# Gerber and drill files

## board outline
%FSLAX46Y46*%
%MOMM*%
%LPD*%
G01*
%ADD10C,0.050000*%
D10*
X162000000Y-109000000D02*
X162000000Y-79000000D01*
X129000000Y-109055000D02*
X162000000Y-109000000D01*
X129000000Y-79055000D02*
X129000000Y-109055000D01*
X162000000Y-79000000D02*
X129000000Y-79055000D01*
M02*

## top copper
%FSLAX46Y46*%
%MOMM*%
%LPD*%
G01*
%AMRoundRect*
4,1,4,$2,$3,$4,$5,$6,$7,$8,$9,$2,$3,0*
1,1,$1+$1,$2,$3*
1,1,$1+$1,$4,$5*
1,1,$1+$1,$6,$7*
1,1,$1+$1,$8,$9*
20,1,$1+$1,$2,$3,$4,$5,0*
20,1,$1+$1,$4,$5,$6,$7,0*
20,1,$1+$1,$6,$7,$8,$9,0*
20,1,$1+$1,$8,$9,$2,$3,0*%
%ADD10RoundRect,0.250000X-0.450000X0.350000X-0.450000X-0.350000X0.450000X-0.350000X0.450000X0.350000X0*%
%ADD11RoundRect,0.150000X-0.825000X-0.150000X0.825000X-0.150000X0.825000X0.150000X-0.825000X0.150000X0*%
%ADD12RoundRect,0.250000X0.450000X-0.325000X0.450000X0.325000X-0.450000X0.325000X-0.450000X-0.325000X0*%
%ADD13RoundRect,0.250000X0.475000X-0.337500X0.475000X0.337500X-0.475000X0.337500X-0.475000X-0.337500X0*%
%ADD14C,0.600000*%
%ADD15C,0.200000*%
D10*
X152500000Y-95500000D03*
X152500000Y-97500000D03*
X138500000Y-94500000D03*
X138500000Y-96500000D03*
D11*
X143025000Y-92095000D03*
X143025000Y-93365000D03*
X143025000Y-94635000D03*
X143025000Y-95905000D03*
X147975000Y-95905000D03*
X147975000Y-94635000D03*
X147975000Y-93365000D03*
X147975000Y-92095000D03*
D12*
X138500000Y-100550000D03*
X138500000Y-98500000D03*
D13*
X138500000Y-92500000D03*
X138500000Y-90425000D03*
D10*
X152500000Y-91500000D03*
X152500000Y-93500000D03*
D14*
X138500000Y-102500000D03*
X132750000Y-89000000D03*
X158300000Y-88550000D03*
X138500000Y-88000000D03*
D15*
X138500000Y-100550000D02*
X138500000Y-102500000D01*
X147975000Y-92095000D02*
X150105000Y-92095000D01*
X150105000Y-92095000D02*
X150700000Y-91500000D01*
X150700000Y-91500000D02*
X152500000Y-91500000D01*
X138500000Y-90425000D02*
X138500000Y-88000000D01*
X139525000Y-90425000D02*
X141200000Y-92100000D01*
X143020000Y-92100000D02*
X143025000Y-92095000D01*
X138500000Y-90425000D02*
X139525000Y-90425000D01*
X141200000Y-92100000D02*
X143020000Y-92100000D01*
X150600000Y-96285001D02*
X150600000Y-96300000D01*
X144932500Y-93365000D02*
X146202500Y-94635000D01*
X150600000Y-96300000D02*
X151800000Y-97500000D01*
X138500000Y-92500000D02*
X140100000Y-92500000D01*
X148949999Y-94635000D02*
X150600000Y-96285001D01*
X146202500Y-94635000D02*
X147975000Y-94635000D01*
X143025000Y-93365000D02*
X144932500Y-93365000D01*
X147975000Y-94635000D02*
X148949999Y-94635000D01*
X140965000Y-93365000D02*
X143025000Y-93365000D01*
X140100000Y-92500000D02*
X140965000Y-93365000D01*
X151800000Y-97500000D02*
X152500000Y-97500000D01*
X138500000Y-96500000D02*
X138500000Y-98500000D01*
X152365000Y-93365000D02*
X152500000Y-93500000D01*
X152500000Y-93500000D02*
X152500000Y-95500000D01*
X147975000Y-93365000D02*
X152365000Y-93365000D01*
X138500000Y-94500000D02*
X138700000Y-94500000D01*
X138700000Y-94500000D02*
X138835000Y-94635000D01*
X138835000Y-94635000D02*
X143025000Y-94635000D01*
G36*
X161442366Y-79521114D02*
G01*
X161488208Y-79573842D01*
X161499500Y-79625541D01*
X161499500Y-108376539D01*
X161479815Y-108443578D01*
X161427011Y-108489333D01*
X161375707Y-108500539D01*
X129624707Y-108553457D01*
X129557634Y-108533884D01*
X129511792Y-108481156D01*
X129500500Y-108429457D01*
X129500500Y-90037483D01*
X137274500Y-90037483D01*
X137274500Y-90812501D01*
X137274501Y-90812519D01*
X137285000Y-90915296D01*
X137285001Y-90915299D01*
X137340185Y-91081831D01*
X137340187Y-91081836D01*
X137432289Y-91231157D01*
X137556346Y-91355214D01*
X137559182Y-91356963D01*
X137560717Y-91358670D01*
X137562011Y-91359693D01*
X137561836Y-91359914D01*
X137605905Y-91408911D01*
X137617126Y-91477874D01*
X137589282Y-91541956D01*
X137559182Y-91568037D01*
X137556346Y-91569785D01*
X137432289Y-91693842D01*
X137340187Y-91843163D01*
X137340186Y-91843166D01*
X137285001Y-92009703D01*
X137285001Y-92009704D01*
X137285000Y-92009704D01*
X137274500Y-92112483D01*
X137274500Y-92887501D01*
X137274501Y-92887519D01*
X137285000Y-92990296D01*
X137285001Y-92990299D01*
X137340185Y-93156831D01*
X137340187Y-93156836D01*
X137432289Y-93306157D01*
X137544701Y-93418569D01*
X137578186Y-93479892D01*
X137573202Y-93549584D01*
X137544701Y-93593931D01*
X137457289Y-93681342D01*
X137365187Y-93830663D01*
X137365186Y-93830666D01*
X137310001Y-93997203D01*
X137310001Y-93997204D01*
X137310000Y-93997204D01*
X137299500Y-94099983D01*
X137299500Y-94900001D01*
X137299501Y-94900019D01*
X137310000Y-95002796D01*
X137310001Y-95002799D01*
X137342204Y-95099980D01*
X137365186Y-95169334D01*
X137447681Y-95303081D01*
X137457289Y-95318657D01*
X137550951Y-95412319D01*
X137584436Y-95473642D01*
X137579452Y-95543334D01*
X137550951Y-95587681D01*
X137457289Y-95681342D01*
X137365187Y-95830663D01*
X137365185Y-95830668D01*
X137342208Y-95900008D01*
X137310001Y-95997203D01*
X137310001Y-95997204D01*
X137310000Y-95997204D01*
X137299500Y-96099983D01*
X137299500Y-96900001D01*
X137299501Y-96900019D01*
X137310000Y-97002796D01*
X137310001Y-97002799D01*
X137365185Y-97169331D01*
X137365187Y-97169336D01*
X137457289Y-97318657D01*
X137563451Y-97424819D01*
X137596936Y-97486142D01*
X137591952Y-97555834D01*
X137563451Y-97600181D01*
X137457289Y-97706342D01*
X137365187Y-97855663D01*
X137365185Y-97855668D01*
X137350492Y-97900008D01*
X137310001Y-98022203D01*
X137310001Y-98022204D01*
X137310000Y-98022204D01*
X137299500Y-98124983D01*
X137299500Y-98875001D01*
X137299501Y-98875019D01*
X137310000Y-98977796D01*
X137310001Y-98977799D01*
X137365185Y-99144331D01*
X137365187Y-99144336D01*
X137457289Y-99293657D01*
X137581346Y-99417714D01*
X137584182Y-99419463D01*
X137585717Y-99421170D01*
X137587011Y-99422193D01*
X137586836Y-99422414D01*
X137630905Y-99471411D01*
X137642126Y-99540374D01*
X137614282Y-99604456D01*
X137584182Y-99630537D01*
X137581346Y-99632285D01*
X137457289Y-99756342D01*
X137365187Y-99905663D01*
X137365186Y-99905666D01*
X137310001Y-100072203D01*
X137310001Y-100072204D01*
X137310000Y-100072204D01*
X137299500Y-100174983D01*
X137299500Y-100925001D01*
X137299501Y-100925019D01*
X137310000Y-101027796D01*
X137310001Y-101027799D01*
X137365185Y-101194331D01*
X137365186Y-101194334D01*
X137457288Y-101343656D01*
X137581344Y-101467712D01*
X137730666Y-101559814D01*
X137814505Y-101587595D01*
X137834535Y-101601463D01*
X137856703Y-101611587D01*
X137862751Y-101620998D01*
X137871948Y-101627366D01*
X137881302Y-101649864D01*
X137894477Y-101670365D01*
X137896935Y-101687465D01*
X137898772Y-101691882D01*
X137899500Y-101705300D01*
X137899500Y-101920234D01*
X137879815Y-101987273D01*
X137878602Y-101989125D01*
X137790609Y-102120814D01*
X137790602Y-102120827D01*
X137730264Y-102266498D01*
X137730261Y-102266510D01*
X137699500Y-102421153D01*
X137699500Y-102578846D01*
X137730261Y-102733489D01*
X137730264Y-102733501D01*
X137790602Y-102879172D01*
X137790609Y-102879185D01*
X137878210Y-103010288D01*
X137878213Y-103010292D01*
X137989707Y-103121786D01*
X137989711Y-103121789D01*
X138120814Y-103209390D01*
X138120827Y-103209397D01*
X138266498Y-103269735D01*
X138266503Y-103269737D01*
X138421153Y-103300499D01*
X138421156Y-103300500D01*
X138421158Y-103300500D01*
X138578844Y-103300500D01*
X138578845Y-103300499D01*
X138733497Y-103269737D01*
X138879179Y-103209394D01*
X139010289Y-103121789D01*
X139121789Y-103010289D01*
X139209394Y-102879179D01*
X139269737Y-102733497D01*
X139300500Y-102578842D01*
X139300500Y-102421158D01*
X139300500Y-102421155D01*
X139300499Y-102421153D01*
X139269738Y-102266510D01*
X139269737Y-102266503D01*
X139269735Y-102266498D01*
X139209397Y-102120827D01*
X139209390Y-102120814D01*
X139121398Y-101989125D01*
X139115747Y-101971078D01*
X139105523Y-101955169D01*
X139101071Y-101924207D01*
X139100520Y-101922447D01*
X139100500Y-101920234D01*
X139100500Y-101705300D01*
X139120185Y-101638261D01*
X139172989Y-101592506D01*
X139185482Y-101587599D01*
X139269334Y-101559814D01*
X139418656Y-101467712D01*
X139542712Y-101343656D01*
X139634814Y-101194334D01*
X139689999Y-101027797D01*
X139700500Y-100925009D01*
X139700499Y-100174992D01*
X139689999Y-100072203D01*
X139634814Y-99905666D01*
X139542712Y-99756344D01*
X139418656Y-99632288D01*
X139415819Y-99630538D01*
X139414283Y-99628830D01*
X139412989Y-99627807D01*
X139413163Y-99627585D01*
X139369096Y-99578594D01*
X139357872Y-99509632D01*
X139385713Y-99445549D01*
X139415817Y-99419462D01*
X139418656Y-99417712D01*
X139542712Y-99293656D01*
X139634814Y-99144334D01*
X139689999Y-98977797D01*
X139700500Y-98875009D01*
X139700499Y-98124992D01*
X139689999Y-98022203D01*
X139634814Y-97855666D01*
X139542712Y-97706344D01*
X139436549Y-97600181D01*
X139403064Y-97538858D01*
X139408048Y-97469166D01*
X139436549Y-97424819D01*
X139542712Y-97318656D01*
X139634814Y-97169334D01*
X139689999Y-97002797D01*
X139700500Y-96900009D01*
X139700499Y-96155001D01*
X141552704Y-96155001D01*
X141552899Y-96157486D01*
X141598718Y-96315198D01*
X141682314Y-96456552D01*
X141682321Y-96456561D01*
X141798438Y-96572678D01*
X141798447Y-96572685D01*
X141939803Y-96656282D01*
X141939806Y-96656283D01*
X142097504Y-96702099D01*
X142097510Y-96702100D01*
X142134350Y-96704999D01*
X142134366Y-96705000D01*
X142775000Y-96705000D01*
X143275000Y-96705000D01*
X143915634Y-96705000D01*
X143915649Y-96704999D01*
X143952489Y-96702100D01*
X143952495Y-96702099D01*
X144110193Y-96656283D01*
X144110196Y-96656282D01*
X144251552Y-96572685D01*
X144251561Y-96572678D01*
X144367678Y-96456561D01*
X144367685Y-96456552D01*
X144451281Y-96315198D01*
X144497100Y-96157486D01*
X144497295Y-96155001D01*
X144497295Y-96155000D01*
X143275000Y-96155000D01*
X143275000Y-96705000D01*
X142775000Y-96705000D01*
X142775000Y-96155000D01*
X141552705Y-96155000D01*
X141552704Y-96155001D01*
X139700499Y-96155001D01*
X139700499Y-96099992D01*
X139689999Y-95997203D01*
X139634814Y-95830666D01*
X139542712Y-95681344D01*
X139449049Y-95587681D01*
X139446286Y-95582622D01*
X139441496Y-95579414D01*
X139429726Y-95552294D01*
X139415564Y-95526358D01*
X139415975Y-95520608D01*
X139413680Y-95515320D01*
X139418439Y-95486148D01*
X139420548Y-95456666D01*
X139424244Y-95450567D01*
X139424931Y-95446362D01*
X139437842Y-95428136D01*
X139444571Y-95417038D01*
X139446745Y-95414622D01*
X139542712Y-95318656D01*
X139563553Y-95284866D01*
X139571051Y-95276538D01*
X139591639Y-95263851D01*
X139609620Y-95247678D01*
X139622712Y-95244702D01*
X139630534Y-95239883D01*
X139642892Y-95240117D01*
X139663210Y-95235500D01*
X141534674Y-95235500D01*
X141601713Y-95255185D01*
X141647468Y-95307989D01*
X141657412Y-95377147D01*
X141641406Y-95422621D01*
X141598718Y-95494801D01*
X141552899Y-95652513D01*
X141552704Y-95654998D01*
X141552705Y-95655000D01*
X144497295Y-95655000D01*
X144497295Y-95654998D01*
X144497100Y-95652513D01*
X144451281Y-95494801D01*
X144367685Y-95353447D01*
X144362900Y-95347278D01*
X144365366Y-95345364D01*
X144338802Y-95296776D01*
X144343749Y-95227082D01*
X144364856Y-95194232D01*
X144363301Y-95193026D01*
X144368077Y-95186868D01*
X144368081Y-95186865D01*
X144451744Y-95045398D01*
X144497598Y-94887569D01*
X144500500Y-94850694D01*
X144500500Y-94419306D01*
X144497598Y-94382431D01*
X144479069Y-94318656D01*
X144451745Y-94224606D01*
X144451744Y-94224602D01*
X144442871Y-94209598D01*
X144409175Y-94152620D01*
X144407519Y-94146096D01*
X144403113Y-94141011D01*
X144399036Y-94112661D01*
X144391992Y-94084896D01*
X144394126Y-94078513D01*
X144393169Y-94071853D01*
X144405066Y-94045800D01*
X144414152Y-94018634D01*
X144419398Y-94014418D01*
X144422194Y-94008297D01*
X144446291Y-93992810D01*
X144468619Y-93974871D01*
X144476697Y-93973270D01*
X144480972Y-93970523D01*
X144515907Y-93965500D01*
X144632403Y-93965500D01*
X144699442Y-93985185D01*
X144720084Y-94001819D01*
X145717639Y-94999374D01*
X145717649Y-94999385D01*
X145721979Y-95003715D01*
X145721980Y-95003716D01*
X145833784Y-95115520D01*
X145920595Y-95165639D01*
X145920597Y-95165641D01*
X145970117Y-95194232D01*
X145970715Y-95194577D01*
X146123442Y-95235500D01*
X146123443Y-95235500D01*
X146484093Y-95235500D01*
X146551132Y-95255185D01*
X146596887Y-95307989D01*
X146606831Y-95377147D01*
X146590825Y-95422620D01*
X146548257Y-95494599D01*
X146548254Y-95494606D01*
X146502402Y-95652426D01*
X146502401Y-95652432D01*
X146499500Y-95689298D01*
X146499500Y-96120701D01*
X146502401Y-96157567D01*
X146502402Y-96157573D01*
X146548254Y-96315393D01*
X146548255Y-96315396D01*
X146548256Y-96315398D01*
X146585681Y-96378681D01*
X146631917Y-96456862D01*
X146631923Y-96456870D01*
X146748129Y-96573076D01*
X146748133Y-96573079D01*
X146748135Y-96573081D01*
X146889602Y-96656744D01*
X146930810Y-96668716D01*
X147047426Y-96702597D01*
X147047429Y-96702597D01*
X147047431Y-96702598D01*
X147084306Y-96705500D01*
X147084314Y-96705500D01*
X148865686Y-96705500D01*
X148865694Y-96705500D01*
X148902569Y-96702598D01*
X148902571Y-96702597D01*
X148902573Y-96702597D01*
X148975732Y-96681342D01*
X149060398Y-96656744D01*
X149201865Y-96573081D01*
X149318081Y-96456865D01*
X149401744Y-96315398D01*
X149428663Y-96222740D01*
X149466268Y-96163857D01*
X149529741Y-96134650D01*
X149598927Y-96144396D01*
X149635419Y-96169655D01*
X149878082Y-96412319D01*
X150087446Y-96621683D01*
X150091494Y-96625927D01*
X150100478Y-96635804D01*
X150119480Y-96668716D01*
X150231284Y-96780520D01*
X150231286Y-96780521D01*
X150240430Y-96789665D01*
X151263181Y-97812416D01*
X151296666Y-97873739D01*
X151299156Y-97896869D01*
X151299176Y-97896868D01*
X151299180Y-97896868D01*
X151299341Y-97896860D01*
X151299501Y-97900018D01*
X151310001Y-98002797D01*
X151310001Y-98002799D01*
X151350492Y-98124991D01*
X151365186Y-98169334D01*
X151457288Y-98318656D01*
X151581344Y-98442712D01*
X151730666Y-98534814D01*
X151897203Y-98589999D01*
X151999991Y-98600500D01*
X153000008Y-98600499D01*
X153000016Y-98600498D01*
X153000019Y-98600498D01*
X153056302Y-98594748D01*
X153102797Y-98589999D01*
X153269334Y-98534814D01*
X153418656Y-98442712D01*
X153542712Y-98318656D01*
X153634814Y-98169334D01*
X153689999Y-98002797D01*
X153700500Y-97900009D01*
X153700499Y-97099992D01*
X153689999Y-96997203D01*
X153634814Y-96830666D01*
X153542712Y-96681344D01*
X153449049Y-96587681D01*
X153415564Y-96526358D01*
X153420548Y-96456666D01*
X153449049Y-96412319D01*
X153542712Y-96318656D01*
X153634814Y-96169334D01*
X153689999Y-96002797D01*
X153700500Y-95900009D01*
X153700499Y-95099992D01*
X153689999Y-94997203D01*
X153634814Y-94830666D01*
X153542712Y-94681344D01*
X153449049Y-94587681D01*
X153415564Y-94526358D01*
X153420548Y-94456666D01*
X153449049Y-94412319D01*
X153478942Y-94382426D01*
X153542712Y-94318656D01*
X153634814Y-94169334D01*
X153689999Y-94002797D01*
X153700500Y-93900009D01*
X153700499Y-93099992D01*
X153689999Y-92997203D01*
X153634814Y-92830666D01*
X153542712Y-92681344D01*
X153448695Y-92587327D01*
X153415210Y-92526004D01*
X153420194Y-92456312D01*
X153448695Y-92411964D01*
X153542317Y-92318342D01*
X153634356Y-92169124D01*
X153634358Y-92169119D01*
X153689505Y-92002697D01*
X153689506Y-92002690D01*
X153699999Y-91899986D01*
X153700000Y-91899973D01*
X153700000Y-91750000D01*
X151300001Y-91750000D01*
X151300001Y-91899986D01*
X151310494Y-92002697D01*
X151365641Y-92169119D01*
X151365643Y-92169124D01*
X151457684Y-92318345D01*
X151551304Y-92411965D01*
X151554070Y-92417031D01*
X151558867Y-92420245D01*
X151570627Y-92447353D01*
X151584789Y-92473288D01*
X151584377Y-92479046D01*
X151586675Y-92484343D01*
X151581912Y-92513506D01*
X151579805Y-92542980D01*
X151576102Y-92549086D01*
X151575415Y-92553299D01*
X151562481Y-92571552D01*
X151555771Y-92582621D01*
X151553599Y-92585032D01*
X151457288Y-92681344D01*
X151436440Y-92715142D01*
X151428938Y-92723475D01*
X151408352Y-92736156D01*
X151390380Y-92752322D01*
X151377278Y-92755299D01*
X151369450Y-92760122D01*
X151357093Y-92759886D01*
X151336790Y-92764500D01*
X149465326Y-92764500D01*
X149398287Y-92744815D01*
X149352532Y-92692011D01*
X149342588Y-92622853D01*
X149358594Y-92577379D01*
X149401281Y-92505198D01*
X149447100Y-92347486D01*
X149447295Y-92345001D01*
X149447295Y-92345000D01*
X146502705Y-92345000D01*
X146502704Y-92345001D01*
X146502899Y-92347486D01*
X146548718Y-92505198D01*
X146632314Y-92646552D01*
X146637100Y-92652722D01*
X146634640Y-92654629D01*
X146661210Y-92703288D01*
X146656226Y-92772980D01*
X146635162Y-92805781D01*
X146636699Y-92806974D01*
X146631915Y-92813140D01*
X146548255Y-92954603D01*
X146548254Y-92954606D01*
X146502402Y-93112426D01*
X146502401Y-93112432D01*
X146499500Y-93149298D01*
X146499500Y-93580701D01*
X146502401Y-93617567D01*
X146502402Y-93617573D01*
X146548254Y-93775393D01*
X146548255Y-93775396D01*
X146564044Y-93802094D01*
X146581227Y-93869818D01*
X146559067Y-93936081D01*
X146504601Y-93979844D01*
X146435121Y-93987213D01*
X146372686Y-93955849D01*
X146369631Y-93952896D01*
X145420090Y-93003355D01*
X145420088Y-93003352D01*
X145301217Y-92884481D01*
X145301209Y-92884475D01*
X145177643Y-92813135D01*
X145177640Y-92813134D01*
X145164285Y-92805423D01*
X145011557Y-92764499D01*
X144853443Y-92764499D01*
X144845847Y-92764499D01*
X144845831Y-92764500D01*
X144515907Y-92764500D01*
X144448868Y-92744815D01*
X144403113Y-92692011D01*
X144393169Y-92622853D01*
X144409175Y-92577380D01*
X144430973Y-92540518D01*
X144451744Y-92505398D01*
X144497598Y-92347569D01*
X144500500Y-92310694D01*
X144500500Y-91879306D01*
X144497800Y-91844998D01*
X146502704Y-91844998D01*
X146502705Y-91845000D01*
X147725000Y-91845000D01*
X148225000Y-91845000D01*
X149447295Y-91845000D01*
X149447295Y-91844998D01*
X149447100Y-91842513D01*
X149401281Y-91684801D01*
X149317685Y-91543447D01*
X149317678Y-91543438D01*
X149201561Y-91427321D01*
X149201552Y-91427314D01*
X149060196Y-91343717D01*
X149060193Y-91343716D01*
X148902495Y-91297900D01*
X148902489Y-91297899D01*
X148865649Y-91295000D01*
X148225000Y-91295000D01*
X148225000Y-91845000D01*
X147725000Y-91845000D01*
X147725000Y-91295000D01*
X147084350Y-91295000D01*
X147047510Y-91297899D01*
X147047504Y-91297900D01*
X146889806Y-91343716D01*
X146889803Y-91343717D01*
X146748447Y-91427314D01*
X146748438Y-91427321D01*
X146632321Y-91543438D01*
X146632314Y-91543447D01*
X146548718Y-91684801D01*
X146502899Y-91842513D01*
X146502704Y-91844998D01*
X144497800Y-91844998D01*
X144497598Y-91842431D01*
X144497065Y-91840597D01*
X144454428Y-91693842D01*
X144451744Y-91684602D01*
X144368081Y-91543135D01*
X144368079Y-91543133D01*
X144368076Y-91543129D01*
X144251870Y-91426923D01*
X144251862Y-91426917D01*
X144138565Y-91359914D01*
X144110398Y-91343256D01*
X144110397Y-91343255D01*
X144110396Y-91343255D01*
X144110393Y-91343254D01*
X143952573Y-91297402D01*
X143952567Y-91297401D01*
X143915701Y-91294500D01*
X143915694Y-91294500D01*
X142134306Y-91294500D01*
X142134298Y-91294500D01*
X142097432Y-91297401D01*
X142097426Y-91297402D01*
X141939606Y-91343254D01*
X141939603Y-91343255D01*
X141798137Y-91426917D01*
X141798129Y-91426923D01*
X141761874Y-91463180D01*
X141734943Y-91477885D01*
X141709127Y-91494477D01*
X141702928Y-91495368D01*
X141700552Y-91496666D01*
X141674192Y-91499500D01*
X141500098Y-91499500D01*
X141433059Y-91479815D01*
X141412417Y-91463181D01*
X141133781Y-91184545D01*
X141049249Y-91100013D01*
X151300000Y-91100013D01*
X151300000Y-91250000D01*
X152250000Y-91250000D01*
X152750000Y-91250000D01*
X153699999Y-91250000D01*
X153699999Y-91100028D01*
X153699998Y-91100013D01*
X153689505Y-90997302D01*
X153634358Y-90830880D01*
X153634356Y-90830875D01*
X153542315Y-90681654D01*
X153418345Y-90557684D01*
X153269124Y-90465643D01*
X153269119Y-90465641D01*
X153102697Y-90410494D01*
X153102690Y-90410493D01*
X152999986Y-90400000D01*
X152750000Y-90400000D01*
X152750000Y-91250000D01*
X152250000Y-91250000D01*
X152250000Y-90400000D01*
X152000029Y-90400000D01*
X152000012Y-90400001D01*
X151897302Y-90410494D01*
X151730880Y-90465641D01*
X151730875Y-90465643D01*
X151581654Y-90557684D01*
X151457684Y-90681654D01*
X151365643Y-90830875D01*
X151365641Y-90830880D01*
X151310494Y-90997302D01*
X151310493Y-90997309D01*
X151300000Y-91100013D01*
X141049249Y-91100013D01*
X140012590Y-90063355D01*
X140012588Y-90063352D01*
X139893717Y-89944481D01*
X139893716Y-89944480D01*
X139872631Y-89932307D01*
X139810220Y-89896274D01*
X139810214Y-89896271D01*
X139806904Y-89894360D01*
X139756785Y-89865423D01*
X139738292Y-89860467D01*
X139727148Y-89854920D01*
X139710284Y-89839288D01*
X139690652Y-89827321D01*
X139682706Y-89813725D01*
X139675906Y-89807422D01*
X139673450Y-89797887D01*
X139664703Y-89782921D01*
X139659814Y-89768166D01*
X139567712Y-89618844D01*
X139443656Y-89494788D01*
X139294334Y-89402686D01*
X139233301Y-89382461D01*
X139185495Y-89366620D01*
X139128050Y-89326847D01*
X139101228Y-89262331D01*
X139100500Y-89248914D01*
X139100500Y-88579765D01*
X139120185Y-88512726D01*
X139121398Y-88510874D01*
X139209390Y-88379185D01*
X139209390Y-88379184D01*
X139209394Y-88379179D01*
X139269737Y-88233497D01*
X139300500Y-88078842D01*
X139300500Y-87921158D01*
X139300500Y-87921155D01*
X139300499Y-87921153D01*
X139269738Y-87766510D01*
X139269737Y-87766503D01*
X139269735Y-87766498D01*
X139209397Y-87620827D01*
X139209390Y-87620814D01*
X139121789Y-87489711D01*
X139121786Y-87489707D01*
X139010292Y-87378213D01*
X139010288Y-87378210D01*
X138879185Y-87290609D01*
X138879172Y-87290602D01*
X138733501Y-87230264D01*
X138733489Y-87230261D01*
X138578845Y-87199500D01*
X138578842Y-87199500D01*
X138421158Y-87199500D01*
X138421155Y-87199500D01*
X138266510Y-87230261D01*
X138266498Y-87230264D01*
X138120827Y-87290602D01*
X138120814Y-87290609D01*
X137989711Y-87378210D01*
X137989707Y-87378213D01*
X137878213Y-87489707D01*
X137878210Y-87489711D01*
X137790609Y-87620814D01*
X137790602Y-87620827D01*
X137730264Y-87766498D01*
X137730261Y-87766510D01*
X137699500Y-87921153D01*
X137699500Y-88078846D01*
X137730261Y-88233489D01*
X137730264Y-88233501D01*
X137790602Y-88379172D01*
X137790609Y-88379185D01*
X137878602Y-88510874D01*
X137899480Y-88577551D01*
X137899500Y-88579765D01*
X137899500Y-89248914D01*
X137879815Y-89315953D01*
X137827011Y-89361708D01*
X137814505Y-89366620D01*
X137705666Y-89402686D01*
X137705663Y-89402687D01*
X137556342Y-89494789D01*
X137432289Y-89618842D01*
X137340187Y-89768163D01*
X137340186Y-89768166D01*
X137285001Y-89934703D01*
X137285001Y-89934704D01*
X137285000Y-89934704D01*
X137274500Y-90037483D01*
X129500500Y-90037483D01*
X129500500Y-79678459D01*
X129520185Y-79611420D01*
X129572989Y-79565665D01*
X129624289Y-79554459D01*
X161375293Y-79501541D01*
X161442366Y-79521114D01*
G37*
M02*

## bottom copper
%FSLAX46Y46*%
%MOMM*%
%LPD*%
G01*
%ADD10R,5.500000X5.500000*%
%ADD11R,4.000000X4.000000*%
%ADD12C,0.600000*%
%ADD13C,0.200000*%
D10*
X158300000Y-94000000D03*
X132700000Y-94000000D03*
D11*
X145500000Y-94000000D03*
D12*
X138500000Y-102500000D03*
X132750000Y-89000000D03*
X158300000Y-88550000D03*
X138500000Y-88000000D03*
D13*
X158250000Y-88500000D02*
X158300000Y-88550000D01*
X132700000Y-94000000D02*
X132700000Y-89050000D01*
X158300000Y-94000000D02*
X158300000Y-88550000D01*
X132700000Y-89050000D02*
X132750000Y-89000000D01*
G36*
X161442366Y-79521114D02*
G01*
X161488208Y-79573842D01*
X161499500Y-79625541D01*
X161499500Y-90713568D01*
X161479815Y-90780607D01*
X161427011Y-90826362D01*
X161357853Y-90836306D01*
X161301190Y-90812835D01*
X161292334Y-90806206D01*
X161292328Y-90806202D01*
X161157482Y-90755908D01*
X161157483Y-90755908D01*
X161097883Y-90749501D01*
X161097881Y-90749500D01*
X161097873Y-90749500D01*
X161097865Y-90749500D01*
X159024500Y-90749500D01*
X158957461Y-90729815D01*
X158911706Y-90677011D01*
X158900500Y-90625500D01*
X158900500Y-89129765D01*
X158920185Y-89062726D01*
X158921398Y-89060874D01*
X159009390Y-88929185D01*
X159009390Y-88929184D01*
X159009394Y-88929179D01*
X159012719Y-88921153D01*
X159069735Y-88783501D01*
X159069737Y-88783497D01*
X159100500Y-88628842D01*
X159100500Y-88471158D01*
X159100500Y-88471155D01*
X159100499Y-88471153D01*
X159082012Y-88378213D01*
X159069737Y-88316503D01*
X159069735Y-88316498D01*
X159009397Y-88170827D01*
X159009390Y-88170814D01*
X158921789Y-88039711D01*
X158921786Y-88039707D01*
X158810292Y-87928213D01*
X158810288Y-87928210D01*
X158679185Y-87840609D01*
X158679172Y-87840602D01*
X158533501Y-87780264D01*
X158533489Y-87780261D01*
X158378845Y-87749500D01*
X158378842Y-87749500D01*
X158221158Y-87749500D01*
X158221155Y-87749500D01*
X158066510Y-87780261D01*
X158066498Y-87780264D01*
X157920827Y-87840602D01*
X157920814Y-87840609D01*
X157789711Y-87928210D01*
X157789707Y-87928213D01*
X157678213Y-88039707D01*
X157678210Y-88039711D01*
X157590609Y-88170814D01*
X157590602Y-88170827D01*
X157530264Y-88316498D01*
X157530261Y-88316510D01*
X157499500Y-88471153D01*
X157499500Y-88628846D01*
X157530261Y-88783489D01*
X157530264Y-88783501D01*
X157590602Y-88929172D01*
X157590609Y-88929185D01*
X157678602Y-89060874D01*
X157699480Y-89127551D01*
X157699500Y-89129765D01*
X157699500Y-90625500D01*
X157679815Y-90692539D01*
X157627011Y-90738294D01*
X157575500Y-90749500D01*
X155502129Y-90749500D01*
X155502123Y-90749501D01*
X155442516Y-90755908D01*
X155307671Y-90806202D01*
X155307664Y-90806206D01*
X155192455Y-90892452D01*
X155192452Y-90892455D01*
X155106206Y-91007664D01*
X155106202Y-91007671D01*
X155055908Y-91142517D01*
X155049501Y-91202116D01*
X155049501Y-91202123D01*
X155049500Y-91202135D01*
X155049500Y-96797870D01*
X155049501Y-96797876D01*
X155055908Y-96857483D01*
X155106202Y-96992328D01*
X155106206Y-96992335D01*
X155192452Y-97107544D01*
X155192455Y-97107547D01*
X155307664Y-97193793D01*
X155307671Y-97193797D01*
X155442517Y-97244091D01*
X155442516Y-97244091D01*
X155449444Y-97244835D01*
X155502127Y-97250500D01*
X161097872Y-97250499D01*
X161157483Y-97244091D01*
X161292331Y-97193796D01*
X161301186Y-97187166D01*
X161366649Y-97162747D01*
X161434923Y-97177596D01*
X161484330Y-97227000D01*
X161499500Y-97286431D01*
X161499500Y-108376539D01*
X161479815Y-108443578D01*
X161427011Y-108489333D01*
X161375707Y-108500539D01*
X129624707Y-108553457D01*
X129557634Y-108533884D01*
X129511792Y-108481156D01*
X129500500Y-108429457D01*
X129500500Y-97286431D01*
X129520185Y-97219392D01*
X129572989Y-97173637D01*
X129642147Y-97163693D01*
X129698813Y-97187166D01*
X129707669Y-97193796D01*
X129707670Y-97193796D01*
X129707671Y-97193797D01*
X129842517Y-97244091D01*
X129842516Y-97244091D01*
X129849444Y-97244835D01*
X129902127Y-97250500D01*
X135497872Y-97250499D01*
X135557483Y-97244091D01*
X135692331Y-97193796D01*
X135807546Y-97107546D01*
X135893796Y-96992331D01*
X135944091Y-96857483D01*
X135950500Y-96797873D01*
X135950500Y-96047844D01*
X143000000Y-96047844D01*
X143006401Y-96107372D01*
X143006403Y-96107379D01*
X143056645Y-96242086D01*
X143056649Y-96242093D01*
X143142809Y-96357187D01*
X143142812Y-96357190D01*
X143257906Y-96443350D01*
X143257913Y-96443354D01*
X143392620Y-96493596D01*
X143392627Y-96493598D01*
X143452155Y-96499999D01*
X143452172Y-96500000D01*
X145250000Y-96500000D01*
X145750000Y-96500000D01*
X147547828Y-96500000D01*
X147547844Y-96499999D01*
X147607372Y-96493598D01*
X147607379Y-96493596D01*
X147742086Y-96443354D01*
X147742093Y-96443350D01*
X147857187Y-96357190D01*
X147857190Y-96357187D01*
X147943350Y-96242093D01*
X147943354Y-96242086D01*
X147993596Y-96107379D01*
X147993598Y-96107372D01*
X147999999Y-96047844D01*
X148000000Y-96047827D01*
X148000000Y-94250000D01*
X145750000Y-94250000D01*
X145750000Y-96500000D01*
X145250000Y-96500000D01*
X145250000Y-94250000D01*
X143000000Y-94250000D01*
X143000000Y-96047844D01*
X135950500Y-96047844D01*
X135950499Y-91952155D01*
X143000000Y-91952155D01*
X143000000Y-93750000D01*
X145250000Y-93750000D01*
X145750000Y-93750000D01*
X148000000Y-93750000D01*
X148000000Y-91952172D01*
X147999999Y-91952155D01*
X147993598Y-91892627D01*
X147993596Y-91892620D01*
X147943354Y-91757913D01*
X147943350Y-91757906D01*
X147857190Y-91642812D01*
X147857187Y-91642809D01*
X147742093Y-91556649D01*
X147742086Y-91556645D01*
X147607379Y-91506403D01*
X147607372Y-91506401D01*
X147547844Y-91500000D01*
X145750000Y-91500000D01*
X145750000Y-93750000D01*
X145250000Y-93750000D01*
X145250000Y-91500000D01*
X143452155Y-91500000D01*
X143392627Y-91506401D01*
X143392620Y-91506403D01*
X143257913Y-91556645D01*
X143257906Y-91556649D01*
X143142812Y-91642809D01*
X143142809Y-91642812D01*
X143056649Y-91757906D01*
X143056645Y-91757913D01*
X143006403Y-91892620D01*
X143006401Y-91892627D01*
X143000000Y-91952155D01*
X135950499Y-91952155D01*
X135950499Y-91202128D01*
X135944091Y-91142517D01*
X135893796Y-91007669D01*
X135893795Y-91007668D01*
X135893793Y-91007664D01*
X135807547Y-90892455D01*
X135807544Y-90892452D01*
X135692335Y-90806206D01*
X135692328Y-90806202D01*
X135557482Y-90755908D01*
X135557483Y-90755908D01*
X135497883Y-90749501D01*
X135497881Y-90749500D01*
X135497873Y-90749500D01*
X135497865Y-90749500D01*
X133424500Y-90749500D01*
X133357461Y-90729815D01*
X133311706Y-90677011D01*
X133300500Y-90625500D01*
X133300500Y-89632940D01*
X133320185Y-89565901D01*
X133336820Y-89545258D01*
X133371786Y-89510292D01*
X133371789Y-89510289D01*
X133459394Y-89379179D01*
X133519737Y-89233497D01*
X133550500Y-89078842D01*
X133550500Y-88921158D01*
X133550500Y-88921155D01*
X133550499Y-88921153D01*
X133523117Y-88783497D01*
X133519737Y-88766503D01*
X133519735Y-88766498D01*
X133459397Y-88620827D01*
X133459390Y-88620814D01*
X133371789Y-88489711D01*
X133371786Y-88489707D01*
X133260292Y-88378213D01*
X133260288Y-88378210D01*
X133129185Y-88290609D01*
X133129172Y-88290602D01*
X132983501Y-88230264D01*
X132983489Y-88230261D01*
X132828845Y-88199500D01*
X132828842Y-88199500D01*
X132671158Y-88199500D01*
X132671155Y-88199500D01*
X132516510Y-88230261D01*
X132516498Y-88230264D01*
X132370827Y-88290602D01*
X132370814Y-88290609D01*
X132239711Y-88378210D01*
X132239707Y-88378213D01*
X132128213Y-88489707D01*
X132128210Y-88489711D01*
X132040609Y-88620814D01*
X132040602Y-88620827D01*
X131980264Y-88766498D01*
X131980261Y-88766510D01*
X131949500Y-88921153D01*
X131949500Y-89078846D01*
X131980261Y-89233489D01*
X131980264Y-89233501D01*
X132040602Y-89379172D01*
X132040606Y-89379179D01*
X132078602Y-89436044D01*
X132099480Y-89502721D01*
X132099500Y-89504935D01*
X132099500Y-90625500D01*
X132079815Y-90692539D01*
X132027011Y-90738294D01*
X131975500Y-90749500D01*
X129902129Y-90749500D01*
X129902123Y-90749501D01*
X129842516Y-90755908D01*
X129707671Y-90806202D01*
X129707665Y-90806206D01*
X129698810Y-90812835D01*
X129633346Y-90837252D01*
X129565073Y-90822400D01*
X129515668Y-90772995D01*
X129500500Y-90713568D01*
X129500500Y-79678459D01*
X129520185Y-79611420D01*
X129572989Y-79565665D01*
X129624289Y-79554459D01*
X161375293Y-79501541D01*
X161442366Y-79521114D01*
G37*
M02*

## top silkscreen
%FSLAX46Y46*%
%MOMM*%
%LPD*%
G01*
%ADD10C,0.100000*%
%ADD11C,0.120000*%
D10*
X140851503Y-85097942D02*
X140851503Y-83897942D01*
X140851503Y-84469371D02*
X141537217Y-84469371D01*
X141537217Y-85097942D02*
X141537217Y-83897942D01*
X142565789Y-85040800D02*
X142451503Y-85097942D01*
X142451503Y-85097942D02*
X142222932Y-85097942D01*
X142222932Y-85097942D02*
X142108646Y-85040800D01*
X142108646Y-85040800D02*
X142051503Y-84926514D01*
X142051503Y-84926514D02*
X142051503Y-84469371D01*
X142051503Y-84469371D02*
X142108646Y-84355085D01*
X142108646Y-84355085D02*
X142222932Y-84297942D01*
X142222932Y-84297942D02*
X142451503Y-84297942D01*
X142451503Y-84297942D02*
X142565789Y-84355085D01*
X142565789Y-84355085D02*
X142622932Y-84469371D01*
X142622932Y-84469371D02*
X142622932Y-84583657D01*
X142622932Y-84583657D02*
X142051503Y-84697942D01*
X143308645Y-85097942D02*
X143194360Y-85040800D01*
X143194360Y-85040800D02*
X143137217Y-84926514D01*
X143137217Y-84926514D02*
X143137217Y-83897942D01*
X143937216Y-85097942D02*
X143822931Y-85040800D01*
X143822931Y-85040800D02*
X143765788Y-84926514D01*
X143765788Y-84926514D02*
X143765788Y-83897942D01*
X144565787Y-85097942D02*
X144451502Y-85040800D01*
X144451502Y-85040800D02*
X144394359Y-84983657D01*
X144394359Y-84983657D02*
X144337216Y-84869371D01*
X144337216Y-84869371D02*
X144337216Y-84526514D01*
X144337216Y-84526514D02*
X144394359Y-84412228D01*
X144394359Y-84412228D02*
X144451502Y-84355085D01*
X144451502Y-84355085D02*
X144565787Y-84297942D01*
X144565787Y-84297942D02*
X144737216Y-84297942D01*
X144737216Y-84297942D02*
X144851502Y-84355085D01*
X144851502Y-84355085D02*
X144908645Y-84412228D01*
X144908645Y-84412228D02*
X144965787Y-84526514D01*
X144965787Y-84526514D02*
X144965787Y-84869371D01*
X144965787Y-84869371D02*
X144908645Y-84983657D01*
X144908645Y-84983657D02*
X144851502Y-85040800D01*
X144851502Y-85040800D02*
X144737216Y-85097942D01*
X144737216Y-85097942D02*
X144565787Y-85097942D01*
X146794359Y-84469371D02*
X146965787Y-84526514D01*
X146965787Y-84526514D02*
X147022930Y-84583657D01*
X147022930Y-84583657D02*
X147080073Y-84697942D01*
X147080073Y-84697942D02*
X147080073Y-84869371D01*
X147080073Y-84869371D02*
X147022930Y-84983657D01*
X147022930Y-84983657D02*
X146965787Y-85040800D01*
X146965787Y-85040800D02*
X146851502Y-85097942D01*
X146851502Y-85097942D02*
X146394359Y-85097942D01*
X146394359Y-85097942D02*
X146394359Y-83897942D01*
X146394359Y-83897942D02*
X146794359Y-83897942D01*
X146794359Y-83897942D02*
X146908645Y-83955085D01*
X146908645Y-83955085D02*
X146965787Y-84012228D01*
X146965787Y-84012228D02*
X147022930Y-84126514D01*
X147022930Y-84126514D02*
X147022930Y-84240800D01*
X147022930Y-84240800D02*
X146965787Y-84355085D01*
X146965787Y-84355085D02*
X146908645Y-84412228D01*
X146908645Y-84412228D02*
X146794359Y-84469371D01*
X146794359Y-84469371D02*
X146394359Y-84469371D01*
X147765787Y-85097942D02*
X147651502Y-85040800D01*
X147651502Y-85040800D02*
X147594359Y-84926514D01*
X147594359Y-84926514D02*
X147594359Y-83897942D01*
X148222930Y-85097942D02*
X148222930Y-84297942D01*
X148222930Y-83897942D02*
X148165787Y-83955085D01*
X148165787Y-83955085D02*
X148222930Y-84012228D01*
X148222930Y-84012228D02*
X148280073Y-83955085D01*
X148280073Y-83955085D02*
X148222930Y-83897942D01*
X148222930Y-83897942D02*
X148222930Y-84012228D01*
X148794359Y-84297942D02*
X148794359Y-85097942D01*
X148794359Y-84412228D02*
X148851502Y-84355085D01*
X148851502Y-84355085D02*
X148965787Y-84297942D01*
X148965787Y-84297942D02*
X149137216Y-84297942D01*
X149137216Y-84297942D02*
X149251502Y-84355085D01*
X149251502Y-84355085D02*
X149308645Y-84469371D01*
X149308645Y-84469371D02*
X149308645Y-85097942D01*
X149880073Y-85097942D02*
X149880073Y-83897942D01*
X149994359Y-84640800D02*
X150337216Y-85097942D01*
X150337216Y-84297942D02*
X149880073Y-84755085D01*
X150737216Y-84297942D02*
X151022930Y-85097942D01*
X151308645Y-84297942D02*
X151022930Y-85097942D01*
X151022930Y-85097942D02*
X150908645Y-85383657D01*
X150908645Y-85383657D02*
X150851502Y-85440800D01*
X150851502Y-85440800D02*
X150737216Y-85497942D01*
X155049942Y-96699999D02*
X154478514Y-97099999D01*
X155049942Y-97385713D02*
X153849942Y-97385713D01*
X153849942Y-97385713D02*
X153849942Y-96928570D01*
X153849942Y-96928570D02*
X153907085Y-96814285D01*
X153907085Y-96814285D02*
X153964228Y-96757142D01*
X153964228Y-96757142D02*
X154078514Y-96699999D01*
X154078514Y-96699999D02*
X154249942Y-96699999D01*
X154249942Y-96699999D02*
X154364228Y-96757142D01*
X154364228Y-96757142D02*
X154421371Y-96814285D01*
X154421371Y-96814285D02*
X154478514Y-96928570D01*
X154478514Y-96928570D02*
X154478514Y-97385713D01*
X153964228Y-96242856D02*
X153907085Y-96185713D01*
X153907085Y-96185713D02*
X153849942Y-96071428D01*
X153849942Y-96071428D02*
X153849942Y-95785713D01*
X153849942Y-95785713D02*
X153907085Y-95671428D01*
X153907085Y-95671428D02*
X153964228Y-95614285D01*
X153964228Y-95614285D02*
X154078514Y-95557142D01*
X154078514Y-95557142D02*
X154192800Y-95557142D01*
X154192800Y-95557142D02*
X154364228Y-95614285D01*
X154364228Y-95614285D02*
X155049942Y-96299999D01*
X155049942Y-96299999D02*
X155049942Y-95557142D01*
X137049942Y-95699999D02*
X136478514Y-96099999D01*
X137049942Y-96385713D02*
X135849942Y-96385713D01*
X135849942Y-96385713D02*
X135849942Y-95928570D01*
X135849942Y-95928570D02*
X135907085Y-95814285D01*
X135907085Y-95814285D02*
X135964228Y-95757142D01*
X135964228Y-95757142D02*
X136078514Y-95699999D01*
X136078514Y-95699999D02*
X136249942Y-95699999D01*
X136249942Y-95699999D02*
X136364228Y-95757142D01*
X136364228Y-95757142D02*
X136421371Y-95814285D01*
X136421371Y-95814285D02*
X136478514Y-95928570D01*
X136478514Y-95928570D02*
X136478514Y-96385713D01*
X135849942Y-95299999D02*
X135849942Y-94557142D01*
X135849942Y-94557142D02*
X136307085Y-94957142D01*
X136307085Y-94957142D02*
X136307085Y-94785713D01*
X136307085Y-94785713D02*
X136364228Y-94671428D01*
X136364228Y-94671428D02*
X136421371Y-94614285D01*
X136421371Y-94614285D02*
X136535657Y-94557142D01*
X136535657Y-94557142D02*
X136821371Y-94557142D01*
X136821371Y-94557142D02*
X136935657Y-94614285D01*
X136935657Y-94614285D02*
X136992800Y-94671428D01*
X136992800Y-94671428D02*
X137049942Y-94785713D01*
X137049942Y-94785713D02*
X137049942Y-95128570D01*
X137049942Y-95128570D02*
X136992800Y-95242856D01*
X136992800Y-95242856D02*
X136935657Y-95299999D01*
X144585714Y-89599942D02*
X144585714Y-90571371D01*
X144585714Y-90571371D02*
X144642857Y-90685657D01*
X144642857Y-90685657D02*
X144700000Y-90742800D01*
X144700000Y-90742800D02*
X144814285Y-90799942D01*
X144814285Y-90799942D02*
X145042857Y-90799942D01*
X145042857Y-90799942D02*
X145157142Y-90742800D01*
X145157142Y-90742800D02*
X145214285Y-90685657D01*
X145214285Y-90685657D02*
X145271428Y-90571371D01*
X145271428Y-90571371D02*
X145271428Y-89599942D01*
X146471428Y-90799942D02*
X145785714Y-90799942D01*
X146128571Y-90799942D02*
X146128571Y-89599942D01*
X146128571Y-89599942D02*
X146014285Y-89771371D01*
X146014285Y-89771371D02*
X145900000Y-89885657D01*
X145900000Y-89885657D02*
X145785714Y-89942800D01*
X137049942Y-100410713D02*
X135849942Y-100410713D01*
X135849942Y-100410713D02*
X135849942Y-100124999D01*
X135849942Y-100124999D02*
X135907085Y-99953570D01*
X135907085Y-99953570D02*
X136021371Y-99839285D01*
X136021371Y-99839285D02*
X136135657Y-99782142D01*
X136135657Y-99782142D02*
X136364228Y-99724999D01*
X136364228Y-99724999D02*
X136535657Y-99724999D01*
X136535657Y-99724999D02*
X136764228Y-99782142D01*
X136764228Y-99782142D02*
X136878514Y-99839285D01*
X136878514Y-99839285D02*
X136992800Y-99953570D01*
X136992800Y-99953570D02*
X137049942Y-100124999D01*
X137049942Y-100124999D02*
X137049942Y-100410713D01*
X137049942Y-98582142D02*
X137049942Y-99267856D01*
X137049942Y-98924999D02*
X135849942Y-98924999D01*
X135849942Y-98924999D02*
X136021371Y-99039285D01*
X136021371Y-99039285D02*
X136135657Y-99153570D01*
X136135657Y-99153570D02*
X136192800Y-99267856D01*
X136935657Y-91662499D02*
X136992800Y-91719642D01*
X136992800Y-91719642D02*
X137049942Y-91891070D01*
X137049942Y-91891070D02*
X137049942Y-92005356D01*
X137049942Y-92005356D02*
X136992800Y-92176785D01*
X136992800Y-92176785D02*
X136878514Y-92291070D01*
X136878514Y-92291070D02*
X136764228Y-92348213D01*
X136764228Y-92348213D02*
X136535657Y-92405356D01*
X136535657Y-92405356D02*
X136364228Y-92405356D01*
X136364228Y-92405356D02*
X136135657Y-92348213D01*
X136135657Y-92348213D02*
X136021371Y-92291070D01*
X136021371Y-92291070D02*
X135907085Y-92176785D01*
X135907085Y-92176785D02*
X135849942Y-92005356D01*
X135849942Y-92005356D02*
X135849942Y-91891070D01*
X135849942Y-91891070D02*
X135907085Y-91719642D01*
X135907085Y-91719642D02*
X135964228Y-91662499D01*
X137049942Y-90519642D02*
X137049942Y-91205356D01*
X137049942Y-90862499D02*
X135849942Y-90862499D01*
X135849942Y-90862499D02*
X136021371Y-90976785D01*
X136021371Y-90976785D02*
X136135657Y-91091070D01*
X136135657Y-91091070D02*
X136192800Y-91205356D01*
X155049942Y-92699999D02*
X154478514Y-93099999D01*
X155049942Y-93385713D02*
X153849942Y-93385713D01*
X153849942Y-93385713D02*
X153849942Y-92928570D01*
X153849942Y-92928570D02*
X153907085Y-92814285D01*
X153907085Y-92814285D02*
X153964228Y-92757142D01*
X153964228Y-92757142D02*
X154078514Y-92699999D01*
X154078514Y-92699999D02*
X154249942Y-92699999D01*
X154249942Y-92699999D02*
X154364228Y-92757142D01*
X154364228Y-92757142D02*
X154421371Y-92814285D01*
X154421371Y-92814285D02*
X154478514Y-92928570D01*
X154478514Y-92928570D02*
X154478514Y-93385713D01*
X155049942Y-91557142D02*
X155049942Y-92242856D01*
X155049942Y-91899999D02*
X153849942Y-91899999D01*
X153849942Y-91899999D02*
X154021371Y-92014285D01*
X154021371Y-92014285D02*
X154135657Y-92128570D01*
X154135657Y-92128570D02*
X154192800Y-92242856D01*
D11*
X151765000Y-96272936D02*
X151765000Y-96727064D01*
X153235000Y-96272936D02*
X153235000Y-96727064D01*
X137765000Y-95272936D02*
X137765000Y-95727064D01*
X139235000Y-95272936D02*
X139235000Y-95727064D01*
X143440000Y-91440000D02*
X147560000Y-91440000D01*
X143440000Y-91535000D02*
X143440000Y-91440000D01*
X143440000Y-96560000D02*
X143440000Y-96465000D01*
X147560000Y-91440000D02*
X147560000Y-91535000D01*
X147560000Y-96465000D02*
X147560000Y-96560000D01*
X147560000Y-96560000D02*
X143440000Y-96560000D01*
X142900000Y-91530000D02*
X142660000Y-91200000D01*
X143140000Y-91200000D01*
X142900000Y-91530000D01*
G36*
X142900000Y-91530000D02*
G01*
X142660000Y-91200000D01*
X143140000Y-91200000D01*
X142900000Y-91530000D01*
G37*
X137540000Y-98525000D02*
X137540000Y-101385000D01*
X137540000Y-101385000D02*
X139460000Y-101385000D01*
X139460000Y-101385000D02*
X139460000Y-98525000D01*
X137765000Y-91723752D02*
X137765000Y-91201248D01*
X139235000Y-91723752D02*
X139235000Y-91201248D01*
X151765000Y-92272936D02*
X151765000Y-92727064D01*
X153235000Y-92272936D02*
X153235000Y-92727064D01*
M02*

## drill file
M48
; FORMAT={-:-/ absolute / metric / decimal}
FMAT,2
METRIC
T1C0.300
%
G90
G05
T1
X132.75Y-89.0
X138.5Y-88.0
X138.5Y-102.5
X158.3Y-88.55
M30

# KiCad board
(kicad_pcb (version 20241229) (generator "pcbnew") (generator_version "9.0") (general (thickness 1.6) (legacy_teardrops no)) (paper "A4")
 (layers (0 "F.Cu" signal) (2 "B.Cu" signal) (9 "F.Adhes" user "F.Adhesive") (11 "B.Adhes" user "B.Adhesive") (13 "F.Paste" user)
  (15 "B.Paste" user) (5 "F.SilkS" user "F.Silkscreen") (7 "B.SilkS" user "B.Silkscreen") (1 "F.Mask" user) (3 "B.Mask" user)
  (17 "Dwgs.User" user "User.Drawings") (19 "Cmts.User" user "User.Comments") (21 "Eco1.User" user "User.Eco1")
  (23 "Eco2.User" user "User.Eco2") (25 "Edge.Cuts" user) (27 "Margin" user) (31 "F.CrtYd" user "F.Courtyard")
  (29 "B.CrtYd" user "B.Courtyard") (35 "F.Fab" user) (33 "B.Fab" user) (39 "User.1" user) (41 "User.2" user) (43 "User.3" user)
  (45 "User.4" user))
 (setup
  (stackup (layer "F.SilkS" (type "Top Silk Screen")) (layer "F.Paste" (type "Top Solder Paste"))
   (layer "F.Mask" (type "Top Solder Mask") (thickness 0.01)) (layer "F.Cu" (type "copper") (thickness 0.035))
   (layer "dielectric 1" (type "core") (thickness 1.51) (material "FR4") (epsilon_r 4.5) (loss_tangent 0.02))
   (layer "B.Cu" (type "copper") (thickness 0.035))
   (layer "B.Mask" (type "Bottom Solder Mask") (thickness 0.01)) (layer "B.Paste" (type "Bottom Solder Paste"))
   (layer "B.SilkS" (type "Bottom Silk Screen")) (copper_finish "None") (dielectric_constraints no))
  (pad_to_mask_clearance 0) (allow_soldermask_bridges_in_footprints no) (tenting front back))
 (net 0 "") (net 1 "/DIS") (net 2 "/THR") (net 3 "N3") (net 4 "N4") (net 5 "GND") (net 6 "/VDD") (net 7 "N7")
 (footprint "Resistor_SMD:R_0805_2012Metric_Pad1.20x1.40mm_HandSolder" (layer "F.Cu") (at 152.5 96.5 -90)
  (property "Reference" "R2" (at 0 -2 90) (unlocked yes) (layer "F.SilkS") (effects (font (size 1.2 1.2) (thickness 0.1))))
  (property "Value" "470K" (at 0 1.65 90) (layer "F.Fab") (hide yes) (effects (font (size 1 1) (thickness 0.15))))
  (fp_line (start -0.227064 0.735) (end 0.227064 0.735) (stroke (width 0.12) (type solid)) (layer "F.SilkS"))
  (fp_line (start -0.227064 -0.735) (end 0.227064 -0.735) (stroke (width 0.12) (type solid)) (layer "F.SilkS"))
  (pad "1" smd roundrect (at -1 0 270) (size 1.2 1.4) (layers "F.Cu" "F.Mask" "F.Paste") (roundrect_rratio 0.208333) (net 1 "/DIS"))
  (pad "2" smd roundrect (at 1 0 270) (size 1.2 1.4) (layers "F.Cu" "F.Mask" "F.Paste") (roundrect_rratio 0.208333) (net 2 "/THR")))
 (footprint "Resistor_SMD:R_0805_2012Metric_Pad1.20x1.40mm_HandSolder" (layer "F.Cu") (at 138.5 95.5 -90)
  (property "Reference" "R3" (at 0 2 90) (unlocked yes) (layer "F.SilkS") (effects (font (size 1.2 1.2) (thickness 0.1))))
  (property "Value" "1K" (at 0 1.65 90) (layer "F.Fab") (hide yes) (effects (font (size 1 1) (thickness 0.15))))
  (fp_line (start -0.227064 0.735) (end 0.227064 0.735) (stroke (width 0.12) (type solid)) (layer "F.SilkS"))
  (fp_line (start -0.227064 -0.735) (end 0.227064 -0.735) (stroke (width 0.12) (type solid)) (layer "F.SilkS"))
  (pad "1" smd roundrect (at -1 0 270) (size 1.2 1.4) (layers "F.Cu" "F.Mask" "F.Paste") (roundrect_rratio 0.208333) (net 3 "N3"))
  (pad "2" smd roundrect (at 1 0 270) (size 1.2 1.4) (layers "F.Cu" "F.Mask" "F.Paste") (roundrect_rratio 0.208333) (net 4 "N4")))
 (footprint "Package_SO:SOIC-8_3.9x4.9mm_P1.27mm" (layer "F.Cu") (at 145.5 94)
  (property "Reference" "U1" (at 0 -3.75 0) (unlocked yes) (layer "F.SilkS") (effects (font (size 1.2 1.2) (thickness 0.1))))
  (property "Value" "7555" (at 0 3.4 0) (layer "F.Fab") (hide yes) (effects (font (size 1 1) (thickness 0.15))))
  (fp_line (start -2.06 -2.56) (end 2.06 -2.56) (stroke (width 0.12) (type solid)) (layer "F.SilkS"))
  (fp_line (start -2.06 -2.465) (end -2.06 -2.56) (stroke (width 0.12) (type solid)) (layer "F.SilkS"))
  (fp_line (start -2.06 2.56) (end -2.06 2.465) (stroke (width 0.12) (type solid)) (layer "F.SilkS"))
  (fp_line (start 2.06 -2.56) (end 2.06 -2.465) (stroke (width 0.12) (type solid)) (layer "F.SilkS"))
  (fp_line (start 2.06 2.465) (end 2.06 2.56) (stroke (width 0.12) (type solid)) (layer "F.SilkS"))
  (fp_line (start 2.06 2.56) (end -2.06 2.56) (stroke (width 0.12) (type solid)) (layer "F.SilkS"))
  (fp_poly (pts (xy -2.6 -2.47) (xy -2.84 -2.8) (xy -2.36 -2.8)) (stroke (width 0.12) (type solid)) (fill yes) (layer "F.SilkS"))
  (pad "1" smd roundrect (at -2.475 -1.905) (size 1.95 0.6) (layers "F.Cu" "F.Mask" "F.Paste") (roundrect_rratio 0.25) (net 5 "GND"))
  (pad "2" smd roundrect (at -2.475 -0.635) (size 1.95 0.6) (layers "F.Cu" "F.Mask" "F.Paste") (roundrect_rratio 0.25) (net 2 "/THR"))
  (pad "3" smd roundrect (at -2.475 0.635) (size 1.95 0.6) (layers "F.Cu" "F.Mask" "F.Paste") (roundrect_rratio 0.25) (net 3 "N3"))
  (pad "4" smd roundrect (at -2.475 1.905) (size 1.95 0.6) (layers "F.Cu" "F.Mask" "F.Paste") (roundrect_rratio 0.25) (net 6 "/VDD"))
  (pad "5" smd roundrect (at 2.475 1.905) (size 1.95 0.6) (layers "F.Cu" "F.Mask" "F.Paste") (roundrect_rratio 0.25) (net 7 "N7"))
  (pad "6" smd roundrect (at 2.475 0.635) (size 1.95 0.6) (layers "F.Cu" "F.Mask" "F.Paste") (roundrect_rratio 0.25) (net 2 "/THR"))
  (pad "7" smd roundrect (at 2.475 -0.635) (size 1.95 0.6) (layers "F.Cu" "F.Mask" "F.Paste") (roundrect_rratio 0.25) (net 1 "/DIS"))
  (pad "8" smd roundrect (at 2.475 -1.905) (size 1.95 0.6) (layers "F.Cu" "F.Mask" "F.Paste") (roundrect_rratio 0.25) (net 6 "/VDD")))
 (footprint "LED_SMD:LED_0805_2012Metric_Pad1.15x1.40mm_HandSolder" (layer "F.Cu") (at 138.5 99.525 90)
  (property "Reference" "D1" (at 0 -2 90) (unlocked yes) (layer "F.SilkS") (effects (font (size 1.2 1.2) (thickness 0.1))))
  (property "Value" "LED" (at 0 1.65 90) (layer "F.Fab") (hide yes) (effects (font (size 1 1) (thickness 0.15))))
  (fp_line (start 1 -0.96) (end -1.86 -0.96) (stroke (width 0.12) (type solid)) (layer "F.SilkS"))
  (fp_line (start -1.86 -0.96) (end -1.86 0.96) (stroke (width 0.12) (type solid)) (layer "F.SilkS"))
  (fp_line (start -1.86 0.96) (end 1 0.96) (stroke (width 0.12) (type solid)) (layer "F.SilkS"))
  (pad "1" smd roundrect (at -1.025 0 90) (size 1.15 1.4) (layers "F.Cu" "F.Mask" "F.Paste") (roundrect_rratio 0.217391) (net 5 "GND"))
  (pad "2" smd roundrect (at 1.025 0 90) (size 1.15 1.4) (layers "F.Cu" "F.Mask" "F.Paste") (roundrect_rratio 0.217391) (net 4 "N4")))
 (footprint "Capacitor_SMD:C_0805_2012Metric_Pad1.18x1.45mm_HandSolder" (layer "F.Cu") (at 138.5 91.4625 90)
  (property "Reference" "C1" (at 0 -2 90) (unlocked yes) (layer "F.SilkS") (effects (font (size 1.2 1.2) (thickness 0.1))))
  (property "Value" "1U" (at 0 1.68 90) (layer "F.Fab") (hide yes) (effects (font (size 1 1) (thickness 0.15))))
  (fp_line (start -0.261252 -0.735) (end 0.261252 -0.735) (stroke (width 0.12) (type solid)) (layer "F.SilkS"))
  (fp_line (start -0.261252 0.735) (end 0.261252 0.735) (stroke (width 0.12) (type solid)) (layer "F.SilkS"))
  (pad "1" smd roundrect (at -1.0375 0 90) (size 1.175 1.45) (layers "F.Cu" "F.Mask" "F.Paste") (roundrect_rratio 0.212766) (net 2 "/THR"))
  (pad "2" smd roundrect (at 1.0375 0 90) (size 1.175 1.45) (layers "F.Cu" "F.Mask" "F.Paste") (roundrect_rratio 0.212766) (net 5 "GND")))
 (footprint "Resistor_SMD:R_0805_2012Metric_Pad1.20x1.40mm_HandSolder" (layer "F.Cu") (at 152.5 92.5 -90)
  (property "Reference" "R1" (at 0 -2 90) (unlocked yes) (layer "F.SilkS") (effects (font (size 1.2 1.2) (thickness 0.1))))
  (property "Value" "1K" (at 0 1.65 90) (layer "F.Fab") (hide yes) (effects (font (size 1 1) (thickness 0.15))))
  (fp_line (start -0.227064 0.735) (end 0.227064 0.735) (stroke (width 0.12) (type solid)) (layer "F.SilkS"))
  (fp_line (start -0.227064 -0.735) (end 0.227064 -0.735) (stroke (width 0.12) (type solid)) (layer "F.SilkS"))
  (pad "1" smd roundrect (at -1 0 270) (size 1.2 1.4) (layers "F.Cu" "F.Mask" "F.Paste") (roundrect_rratio 0.208333) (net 6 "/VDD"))
  (pad "2" smd roundrect (at 1 0 270) (size 1.2 1.4) (layers "F.Cu" "F.Mask" "F.Paste") (roundrect_rratio 0.208333) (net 1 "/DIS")))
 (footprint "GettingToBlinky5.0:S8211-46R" (layer "B.Cu") (at 145.5 94 180)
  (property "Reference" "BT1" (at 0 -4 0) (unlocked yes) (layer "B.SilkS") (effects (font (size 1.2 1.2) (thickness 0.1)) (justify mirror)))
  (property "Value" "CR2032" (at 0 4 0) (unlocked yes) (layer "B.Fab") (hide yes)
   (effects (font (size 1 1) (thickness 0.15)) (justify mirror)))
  (pad "1" smd rect (at -12.8 0 180) (size 5.5 5.5) (layers "B.Cu" "B.Mask" "B.Paste") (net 6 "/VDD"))
  (pad "1" smd rect (at 12.8 0 180) (size 5.5 5.5) (layers "B.Cu" "B.Mask" "B.Paste") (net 6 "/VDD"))
  (pad "2" smd rect (at 0 0 180) (size 4 4) (layers "B.Cu" "B.Mask" "B.Paste") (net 5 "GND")))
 (gr_line (start 162 109) (end 162 79) (stroke (width 0.05) (type default)) (layer "Edge.Cuts"))
 (gr_line (start 129 109.055) (end 162 109) (stroke (width 0.05) (type default)) (layer "Edge.Cuts"))
 (gr_line (start 129 79.055) (end 129 109.055) (stroke (width 0.05) (type default)) (layer "Edge.Cuts"))
 (gr_line (start 162 79) (end 129 79.055) (stroke (width 0.05) (type default)) (layer "Edge.Cuts"))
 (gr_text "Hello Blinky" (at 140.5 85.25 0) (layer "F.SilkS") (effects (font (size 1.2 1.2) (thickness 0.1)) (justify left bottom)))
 (segment (start 147.975 92.095) (end 150.105 92.095) (width 0.2) (layer "F.Cu") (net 6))
 (segment (start 150.105 92.095) (end 150.7 91.5) (width 0.2) (layer "F.Cu") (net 6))
 (segment (start 150.7 91.5) (end 152.5 91.5) (width 0.2) (layer "F.Cu") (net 6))
 (via (at 132.75 89) (size 0.6) (drill 0.3) (layers "F.Cu" "B.Cu") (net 6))
 (via (at 158.3 88.55) (size 0.6) (drill 0.3) (layers "F.Cu" "B.Cu") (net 6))
 (segment (start 158.25 88.5) (end 158.3 88.55) (width 0.2) (layer "B.Cu") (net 6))
 (segment (start 132.7 94) (end 132.7 89.05) (width 0.2) (layer "B.Cu") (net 6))
 (segment (start 158.3 94) (end 158.3 88.55) (width 0.2) (layer "B.Cu") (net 6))
 (segment (start 132.7 89.05) (end 132.75 89) (width 0.2) (layer "B.Cu") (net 6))
 (segment (start 138.5 90.425) (end 138.5 88) (width 0.2) (layer "F.Cu") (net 5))
 (segment (start 139.525 90.425) (end 141.2 92.1) (width 0.2) (layer "F.Cu") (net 5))
 (segment (start 138.5 100.55) (end 138.5 102.5) (width 0.2) (layer "F.Cu") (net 5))
 (segment (start 143.02 92.1) (end 143.025 92.095) (width 0.2) (layer "F.Cu") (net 5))
 (segment (start 138.5 90.425) (end 139.525 90.425) (width 0.2) (layer "F.Cu") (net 5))
 (segment (start 141.2 92.1) (end 143.02 92.1) (width 0.2) (layer "F.Cu") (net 5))
 (via (at 138.5 88) (size 0.6) (drill 0.3) (layers "F.Cu" "B.Cu") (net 5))
 (via (at 138.5 102.5) (size 0.6) (drill 0.3) (layers "F.Cu" "B.Cu") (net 5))
 (segment (start 150.6 96.285001) (end 150.6 96.3) (width 0.2) (layer "F.Cu") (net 2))
 (segment (start 144.9325 93.365) (end 146.2025 94.635) (width 0.2) (layer "F.Cu") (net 2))
 (segment (start 150.6 96.3) (end 151.8 97.5) (width 0.2) (layer "F.Cu") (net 2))
 (segment (start 138.5 92.5) (end 140.1 92.5) (width 0.2) (layer "F.Cu") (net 2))
 (segment (start 148.949999 94.635) (end 150.6 96.285001) (width 0.2) (layer "F.Cu") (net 2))
 (segment (start 146.2025 94.635) (end 147.975 94.635) (width 0.2) (layer "F.Cu") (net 2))
 (segment (start 143.025 93.365) (end 144.9325 93.365) (width 0.2) (layer "F.Cu") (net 2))
 (segment (start 147.975 94.635) (end 148.949999 94.635) (width 0.2) (layer "F.Cu") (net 2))
 (segment (start 140.965 93.365) (end 143.025 93.365) (width 0.2) (layer "F.Cu") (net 2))
 (segment (start 140.1 92.5) (end 140.965 93.365) (width 0.2) (layer "F.Cu") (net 2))
 (segment (start 151.8 97.5) (end 152.5 97.5) (width 0.2) (layer "F.Cu") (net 2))
 (segment (start 138.5 96.5) (end 138.5 98.5) (width 0.2) (layer "F.Cu") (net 4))
 (segment (start 152.365 93.365) (end 152.5 93.5) (width 0.2) (layer "F.Cu") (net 1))
 (segment (start 152.5 93.5) (end 152.5 95.5) (width 0.2) (layer "F.Cu") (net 1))
 (segment (start 147.975 93.365) (end 152.365 93.365) (width 0.2) (layer "F.Cu") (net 1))
 (segment (start 138.5 94.5) (end 138.7 94.5) (width 0.2) (layer "F.Cu") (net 3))
 (segment (start 138.7 94.5) (end 138.835 94.635) (width 0.2) (layer "F.Cu") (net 3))
 (segment (start 138.835 94.635) (end 143.025 94.635) (width 0.2) (layer "F.Cu") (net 3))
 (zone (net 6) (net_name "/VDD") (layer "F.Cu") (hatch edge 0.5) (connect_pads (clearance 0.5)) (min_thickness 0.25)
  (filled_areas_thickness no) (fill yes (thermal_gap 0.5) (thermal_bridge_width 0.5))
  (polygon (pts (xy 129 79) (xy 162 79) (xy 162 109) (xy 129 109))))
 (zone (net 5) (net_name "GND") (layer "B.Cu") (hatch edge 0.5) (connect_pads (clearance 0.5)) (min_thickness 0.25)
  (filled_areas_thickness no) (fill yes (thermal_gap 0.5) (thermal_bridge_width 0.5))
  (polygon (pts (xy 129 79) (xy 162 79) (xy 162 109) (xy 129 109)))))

